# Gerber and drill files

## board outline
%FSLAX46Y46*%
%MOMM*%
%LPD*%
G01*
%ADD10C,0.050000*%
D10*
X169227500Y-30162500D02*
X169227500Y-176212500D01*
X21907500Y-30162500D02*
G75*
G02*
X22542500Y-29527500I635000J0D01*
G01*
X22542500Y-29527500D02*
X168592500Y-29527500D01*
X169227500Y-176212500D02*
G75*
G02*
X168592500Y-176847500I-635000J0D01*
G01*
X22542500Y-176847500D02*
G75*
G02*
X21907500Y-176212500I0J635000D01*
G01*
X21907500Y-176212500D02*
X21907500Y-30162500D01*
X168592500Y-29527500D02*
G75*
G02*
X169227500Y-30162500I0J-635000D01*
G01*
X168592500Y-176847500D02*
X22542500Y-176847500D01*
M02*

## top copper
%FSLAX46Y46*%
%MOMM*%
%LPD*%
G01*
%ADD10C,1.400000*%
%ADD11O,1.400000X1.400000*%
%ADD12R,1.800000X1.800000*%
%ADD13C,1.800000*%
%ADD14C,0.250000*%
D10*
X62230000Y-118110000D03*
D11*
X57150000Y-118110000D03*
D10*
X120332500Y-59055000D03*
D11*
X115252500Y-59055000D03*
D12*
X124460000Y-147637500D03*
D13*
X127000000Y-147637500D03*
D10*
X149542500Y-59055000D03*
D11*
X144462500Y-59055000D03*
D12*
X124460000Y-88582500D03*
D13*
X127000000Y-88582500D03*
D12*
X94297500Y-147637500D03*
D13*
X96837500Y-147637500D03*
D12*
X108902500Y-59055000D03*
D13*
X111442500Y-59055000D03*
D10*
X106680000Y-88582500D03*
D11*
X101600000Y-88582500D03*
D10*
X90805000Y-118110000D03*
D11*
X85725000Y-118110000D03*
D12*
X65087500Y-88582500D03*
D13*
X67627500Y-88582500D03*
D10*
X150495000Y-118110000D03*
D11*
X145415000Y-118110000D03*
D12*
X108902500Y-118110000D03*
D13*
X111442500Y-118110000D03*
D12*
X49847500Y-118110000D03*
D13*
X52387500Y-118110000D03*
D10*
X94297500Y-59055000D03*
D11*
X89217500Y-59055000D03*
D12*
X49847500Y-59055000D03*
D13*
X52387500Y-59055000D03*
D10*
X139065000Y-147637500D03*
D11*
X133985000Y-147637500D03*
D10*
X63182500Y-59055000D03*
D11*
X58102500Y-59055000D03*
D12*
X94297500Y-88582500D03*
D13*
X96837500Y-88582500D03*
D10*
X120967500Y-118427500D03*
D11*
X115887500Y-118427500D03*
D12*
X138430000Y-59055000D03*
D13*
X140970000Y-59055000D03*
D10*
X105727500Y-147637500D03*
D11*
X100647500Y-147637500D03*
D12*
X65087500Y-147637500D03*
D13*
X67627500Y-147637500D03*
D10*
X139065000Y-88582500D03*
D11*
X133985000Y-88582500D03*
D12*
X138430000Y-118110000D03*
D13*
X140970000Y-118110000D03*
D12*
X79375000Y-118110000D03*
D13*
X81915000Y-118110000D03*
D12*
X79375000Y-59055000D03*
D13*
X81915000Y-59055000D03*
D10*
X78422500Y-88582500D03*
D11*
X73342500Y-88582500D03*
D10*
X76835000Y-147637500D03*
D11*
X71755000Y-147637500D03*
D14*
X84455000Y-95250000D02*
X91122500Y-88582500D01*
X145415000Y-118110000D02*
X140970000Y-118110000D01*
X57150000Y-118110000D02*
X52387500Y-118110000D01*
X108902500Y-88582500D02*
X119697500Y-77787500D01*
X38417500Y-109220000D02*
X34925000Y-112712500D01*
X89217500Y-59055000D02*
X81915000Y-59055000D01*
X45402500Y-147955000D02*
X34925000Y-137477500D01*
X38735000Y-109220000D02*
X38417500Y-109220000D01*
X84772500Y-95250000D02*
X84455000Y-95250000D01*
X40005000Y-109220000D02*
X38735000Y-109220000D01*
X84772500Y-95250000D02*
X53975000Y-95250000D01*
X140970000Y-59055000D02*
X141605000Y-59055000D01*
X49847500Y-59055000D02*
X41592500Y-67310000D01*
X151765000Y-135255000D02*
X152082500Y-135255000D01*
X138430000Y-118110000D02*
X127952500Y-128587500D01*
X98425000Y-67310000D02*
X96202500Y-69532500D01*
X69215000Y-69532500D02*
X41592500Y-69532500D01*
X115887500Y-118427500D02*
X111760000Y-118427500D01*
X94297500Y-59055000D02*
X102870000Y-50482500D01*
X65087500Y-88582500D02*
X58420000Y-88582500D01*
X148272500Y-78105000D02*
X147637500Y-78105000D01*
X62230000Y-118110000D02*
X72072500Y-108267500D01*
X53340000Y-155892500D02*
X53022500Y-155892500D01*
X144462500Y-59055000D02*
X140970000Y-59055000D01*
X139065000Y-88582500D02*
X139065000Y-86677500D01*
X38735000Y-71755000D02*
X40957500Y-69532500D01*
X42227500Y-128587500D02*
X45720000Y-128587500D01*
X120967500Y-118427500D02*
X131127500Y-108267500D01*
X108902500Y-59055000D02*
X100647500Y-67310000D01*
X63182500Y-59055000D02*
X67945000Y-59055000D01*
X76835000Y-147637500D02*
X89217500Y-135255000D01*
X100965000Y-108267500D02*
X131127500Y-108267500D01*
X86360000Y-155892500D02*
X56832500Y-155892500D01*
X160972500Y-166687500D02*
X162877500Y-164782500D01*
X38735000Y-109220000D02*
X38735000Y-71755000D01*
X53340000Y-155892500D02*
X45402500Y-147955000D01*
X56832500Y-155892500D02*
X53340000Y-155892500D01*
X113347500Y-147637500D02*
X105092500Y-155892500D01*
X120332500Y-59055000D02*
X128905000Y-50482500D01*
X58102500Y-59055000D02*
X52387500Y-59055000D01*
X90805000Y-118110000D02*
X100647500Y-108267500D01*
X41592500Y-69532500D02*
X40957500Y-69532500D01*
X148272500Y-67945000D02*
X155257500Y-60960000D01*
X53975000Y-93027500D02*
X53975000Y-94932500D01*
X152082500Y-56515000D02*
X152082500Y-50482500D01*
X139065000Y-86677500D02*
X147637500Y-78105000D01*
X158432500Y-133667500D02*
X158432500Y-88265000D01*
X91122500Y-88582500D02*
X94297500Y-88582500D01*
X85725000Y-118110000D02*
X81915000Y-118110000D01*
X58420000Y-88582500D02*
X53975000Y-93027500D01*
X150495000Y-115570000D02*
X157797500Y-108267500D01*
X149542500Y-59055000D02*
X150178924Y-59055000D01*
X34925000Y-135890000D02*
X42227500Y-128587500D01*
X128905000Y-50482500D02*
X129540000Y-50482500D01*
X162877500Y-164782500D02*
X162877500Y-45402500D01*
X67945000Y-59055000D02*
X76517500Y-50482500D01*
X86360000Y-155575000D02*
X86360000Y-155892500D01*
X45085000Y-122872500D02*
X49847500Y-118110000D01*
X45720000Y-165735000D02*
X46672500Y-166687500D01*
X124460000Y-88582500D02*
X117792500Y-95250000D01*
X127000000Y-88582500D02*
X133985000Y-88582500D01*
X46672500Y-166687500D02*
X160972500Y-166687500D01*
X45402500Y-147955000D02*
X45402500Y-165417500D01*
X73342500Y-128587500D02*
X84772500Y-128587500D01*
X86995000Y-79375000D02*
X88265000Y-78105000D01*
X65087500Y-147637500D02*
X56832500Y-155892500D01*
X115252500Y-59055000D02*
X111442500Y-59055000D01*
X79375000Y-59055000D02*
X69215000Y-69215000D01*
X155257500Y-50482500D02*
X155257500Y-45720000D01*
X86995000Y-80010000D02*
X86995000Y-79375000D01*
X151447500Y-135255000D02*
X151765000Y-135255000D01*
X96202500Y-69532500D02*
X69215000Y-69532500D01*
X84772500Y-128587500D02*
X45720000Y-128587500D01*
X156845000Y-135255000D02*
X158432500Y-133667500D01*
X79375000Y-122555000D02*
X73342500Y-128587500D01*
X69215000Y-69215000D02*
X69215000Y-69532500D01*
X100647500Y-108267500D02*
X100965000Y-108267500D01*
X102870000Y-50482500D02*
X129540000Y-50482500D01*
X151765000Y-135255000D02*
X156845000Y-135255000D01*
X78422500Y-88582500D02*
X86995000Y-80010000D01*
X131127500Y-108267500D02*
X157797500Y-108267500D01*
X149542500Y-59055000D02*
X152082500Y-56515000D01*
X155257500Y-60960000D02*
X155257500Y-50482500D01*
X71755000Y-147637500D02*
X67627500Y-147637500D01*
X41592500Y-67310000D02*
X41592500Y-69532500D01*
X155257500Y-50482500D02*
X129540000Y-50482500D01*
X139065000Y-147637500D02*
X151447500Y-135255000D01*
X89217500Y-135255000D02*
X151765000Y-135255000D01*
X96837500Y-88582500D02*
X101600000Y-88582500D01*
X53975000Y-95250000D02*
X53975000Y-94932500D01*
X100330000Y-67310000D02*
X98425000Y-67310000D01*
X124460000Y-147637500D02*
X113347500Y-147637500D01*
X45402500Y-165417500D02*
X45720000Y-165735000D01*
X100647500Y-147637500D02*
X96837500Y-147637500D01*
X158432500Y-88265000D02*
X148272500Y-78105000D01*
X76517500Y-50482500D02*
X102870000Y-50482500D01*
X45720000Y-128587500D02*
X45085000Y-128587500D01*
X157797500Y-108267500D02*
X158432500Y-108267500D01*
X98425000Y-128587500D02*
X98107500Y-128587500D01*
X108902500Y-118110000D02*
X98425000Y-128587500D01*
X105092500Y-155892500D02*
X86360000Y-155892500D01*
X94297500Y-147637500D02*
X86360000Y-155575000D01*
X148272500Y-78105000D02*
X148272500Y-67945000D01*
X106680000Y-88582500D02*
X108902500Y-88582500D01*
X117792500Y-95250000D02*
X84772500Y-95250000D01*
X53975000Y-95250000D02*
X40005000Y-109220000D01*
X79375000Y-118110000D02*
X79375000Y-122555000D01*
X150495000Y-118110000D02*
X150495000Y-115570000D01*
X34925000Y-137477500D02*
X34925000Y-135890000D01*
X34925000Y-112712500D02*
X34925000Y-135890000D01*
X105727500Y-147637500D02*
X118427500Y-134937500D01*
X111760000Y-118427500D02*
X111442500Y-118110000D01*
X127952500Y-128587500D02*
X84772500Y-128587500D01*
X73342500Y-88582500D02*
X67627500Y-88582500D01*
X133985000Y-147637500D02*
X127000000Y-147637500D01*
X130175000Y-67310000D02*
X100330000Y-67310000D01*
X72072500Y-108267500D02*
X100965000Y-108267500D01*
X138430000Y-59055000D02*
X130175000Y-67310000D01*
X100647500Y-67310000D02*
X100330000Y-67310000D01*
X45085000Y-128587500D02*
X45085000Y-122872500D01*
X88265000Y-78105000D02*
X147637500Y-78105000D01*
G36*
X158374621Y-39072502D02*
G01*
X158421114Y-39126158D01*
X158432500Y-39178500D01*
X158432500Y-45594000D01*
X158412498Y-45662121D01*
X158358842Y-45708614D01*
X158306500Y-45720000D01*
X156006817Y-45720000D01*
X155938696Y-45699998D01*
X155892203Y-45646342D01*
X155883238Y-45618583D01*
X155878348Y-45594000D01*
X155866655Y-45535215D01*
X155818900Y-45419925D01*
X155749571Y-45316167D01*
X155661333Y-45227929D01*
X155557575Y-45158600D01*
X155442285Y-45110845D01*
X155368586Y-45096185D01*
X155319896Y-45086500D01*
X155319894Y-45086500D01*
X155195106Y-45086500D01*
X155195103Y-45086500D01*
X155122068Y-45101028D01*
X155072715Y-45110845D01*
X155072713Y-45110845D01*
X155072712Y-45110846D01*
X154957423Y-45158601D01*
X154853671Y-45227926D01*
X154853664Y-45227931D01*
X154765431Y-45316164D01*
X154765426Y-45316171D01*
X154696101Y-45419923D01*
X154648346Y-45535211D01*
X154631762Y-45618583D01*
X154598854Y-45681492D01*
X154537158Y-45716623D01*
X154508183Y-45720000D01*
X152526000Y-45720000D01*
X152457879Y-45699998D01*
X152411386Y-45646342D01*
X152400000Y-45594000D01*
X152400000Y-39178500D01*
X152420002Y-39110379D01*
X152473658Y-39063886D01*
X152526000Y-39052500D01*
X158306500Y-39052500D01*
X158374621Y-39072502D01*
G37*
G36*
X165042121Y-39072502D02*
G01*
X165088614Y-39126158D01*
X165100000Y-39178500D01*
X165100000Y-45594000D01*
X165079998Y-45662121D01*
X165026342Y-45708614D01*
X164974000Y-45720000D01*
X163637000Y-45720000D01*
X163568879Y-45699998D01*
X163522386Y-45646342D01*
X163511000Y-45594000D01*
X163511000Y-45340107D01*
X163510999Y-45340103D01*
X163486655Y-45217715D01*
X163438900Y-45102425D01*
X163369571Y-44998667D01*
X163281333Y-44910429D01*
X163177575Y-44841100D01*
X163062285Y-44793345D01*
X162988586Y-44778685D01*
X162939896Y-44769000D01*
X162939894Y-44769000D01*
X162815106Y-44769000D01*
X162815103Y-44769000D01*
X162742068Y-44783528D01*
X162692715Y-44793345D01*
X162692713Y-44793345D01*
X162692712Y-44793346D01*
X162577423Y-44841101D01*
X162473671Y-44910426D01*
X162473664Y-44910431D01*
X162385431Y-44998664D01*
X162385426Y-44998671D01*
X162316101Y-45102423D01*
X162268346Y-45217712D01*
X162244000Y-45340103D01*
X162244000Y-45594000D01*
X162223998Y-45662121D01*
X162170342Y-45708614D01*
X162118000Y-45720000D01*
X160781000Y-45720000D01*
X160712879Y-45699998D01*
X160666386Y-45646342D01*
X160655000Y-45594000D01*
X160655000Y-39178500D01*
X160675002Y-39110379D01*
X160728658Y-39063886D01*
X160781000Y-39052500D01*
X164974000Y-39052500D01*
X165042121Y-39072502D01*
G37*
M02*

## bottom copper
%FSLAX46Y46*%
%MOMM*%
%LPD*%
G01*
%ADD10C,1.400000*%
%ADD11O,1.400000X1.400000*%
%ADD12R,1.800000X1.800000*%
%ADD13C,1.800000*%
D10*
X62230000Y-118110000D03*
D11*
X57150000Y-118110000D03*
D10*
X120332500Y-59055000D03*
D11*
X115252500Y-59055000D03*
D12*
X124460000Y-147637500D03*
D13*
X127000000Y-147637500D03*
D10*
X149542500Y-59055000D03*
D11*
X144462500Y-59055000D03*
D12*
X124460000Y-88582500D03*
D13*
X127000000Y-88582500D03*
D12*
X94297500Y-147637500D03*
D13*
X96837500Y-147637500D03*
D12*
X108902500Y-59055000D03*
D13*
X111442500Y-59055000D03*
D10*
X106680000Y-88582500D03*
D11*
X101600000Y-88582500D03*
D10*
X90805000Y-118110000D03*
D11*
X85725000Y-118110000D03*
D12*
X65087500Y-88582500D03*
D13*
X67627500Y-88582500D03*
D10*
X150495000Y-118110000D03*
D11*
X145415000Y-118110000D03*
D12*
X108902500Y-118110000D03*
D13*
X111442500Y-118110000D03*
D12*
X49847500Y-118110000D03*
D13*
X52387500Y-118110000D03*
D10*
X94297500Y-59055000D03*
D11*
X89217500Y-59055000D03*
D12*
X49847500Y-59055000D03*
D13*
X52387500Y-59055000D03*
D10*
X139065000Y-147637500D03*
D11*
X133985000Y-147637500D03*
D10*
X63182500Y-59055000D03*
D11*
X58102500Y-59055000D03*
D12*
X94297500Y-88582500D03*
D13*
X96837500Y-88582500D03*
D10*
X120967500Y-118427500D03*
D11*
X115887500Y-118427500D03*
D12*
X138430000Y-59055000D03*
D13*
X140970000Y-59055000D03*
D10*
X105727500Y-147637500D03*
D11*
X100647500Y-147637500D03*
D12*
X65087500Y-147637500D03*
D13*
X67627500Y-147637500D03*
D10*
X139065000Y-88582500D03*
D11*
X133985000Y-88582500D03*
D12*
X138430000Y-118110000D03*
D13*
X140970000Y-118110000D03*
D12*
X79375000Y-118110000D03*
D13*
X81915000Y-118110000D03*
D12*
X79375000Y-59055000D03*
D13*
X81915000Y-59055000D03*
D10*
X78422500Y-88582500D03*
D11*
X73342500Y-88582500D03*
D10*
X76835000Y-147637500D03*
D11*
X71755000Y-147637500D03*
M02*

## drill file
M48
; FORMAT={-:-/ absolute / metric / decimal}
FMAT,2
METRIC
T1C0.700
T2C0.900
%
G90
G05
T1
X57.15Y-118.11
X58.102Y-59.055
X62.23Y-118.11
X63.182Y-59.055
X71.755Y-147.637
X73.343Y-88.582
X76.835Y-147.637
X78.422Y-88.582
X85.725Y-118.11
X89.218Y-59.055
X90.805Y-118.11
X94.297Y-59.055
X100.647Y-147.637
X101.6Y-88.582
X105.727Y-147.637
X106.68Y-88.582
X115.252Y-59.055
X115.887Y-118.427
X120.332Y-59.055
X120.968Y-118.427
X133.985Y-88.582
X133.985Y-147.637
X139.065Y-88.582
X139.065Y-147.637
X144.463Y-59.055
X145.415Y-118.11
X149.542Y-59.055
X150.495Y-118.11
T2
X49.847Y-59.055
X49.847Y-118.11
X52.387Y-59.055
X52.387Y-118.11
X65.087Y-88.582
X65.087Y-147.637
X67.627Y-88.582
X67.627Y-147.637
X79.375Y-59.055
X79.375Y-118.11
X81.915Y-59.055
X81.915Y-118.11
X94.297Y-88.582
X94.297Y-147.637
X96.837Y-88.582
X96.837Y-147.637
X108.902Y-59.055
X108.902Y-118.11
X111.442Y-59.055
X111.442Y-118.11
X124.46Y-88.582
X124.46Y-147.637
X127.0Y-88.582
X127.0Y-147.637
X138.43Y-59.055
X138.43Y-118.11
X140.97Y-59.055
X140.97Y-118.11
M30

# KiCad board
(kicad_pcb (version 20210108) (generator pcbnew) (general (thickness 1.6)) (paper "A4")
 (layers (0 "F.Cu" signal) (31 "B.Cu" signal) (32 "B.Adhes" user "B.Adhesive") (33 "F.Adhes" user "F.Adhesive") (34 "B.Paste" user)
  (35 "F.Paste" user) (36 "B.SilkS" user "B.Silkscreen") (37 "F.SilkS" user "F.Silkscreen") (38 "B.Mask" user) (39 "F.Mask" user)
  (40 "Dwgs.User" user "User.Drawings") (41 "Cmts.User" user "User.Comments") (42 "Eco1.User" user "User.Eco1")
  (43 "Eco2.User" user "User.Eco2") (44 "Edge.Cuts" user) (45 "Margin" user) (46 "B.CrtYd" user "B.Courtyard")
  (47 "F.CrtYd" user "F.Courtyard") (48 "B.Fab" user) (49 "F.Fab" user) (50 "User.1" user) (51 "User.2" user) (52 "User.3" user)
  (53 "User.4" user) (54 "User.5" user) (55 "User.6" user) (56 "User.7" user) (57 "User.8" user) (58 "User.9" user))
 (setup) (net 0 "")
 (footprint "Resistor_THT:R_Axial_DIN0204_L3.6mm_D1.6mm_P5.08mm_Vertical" (layer "F.Cu") (at 62.23 118.11 180)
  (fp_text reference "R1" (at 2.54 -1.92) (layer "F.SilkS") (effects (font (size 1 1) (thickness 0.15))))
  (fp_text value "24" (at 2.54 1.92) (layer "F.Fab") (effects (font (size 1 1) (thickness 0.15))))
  (pad "1" thru_hole circle (at 0 0 180) (locked) (size 1.4 1.4) (drill 0.7) (layers *.Cu *.Mask))
  (pad "2" thru_hole oval (at 5.08 0 180) (locked) (size 1.4 1.4) (drill 0.7) (layers *.Cu *.Mask)))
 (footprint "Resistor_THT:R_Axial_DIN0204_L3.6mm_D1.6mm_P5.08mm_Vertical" (layer "F.Cu") (at 120.3325 59.055 180)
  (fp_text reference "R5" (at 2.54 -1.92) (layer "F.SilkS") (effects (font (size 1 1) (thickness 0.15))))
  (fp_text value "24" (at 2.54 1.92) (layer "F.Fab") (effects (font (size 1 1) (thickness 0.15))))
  (pad "1" thru_hole circle (at 0 0 180) (locked) (size 1.4 1.4) (drill 0.7) (layers *.Cu *.Mask))
  (pad "2" thru_hole oval (at 5.08 0 180) (locked) (size 1.4 1.4) (drill 0.7) (layers *.Cu *.Mask)))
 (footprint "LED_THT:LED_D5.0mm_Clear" (layer "F.Cu") (at 124.46 147.6375)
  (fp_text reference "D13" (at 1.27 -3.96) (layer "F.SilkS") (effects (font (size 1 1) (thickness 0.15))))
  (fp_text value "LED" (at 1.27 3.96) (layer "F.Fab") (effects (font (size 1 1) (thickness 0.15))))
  (pad "1" thru_hole rect (at 0 0) (locked) (size 1.8 1.8) (drill 0.9) (layers *.Cu *.Mask))
  (pad "2" thru_hole circle (at 2.54 0) (locked) (size 1.8 1.8) (drill 0.9) (layers *.Cu *.Mask)))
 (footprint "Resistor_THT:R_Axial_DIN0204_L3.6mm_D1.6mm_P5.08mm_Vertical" (layer "F.Cu") (at 149.5425 59.055 180)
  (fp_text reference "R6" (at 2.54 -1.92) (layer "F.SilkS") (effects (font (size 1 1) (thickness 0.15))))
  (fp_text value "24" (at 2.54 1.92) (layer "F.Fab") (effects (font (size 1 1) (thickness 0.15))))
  (pad "1" thru_hole circle (at 0 0 180) (locked) (size 1.4 1.4) (drill 0.7) (layers *.Cu *.Mask))
  (pad "2" thru_hole oval (at 5.08 0 180) (locked) (size 1.4 1.4) (drill 0.7) (layers *.Cu *.Mask)))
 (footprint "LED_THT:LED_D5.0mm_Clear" (layer "F.Cu") (at 124.46 88.5825)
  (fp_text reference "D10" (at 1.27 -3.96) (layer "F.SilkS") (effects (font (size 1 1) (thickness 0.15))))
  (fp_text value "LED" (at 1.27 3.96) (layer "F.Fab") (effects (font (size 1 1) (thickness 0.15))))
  (pad "1" thru_hole rect (at 0 0) (locked) (size 1.8 1.8) (drill 0.9) (layers *.Cu *.Mask))
  (pad "2" thru_hole circle (at 2.54 0) (locked) (size 1.8 1.8) (drill 0.9) (layers *.Cu *.Mask)))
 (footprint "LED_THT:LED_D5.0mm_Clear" (layer "F.Cu") (at 94.2975 147.6375)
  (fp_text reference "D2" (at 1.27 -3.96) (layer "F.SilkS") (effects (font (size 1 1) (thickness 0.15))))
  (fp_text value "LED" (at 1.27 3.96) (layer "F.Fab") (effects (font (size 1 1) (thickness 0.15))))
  (pad "1" thru_hole rect (at 0 0) (locked) (size 1.8 1.8) (drill 0.9) (layers *.Cu *.Mask))
  (pad "2" thru_hole circle (at 2.54 0) (locked) (size 1.8 1.8) (drill 0.9) (layers *.Cu *.Mask)))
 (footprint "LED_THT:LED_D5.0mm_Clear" (layer "F.Cu") (at 108.9025 59.055)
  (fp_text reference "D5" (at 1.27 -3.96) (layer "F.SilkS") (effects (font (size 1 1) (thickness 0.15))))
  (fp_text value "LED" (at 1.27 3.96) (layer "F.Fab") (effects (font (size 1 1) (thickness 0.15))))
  (pad "1" thru_hole rect (at 0 0) (locked) (size 1.8 1.8) (drill 0.9) (layers *.Cu *.Mask))
  (pad "2" thru_hole circle (at 2.54 0) (locked) (size 1.8 1.8) (drill 0.9) (layers *.Cu *.Mask)))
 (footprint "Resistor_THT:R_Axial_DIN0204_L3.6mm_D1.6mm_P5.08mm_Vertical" (layer "F.Cu") (at 106.68 88.5825 180)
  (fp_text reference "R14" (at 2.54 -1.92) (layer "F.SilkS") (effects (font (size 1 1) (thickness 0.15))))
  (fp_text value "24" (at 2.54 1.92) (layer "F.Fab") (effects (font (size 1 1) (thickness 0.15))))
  (pad "1" thru_hole circle (at 0 0 180) (locked) (size 1.4 1.4) (drill 0.7) (layers *.Cu *.Mask))
  (pad "2" thru_hole oval (at 5.08 0 180) (locked) (size 1.4 1.4) (drill 0.7) (layers *.Cu *.Mask)))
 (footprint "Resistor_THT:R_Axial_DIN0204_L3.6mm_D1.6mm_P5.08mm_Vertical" (layer "F.Cu") (at 90.805 118.11 180)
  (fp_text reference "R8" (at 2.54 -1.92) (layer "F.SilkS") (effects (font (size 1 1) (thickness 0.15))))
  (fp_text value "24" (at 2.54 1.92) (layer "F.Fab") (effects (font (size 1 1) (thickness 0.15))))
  (pad "1" thru_hole circle (at 0 0 180) (locked) (size 1.4 1.4) (drill 0.7) (layers *.Cu *.Mask))
  (pad "2" thru_hole oval (at 5.08 0 180) (locked) (size 1.4 1.4) (drill 0.7) (layers *.Cu *.Mask)))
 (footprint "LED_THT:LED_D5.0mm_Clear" (layer "F.Cu") (at 65.0875 88.5825)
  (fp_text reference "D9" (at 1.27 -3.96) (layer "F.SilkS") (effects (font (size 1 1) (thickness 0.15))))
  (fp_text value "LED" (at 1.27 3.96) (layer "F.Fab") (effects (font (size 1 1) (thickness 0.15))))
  (pad "1" thru_hole rect (at 0 0) (locked) (size 1.8 1.8) (drill 0.9) (layers *.Cu *.Mask))
  (pad "2" thru_hole circle (at 2.54 0) (locked) (size 1.8 1.8) (drill 0.9) (layers *.Cu *.Mask)))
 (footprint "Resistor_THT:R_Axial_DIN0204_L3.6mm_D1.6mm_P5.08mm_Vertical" (layer "F.Cu") (at 150.495 118.11 180)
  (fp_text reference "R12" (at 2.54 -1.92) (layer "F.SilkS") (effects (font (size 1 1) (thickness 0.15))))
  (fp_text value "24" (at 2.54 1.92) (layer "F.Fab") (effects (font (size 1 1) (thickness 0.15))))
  (pad "1" thru_hole circle (at 0 0 180) (locked) (size 1.4 1.4) (drill 0.7) (layers *.Cu *.Mask))
  (pad "2" thru_hole oval (at 5.08 0 180) (locked) (size 1.4 1.4) (drill 0.7) (layers *.Cu *.Mask)))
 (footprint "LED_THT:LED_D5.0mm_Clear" (layer "F.Cu") (at 108.9025 118.11)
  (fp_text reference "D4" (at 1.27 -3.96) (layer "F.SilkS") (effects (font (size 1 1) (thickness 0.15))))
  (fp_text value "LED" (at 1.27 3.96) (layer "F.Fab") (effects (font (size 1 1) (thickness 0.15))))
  (pad "1" thru_hole rect (at 0 0) (locked) (size 1.8 1.8) (drill 0.9) (layers *.Cu *.Mask))
  (pad "2" thru_hole circle (at 2.54 0) (locked) (size 1.8 1.8) (drill 0.9) (layers *.Cu *.Mask)))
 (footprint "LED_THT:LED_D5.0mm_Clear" (layer "F.Cu") (at 49.8475 118.11)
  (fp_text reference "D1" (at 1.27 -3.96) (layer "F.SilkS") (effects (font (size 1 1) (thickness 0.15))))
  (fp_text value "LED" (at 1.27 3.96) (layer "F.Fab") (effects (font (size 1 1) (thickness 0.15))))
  (pad "1" thru_hole rect (at 0 0) (locked) (size 1.8 1.8) (drill 0.9) (layers *.Cu *.Mask))
  (pad "2" thru_hole circle (at 2.54 0) (locked) (size 1.8 1.8) (drill 0.9) (layers *.Cu *.Mask)))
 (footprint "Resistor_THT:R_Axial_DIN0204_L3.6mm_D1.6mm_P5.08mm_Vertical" (layer "F.Cu") (at 94.2975 59.055 180)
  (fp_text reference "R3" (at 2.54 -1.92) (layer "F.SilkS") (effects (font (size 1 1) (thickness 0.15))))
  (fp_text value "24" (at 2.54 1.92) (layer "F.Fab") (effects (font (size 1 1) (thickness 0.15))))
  (pad "1" thru_hole circle (at 0 0 180) (locked) (size 1.4 1.4) (drill 0.7) (layers *.Cu *.Mask))
  (pad "2" thru_hole oval (at 5.08 0 180) (locked) (size 1.4 1.4) (drill 0.7) (layers *.Cu *.Mask)))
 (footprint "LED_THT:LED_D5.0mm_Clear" (layer "F.Cu") (at 49.8475 59.055)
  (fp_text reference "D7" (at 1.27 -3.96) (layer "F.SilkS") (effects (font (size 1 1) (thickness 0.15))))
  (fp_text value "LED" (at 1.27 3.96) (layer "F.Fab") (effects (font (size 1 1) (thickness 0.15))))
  (pad "1" thru_hole rect (at 0 0) (locked) (size 1.8 1.8) (drill 0.9) (layers *.Cu *.Mask))
  (pad "2" thru_hole circle (at 2.54 0) (locked) (size 1.8 1.8) (drill 0.9) (layers *.Cu *.Mask)))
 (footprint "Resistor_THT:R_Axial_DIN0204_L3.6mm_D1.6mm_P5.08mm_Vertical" (layer "F.Cu") (at 139.065 147.6375 180)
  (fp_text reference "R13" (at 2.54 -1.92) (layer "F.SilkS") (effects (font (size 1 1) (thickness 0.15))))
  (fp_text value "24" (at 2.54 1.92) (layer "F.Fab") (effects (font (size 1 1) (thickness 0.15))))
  (pad "1" thru_hole circle (at 0 0 180) (locked) (size 1.4 1.4) (drill 0.7) (layers *.Cu *.Mask))
  (pad "2" thru_hole oval (at 5.08 0 180) (locked) (size 1.4 1.4) (drill 0.7) (layers *.Cu *.Mask)))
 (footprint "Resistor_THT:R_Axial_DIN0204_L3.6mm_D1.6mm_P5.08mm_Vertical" (layer "F.Cu") (at 63.1825 59.055 180)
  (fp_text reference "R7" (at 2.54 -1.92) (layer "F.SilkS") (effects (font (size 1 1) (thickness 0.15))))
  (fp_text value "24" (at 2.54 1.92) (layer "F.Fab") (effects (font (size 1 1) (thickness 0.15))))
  (pad "1" thru_hole circle (at 0 0 180) (locked) (size 1.4 1.4) (drill 0.7) (layers *.Cu *.Mask))
  (pad "2" thru_hole oval (at 5.08 0 180) (locked) (size 1.4 1.4) (drill 0.7) (layers *.Cu *.Mask)))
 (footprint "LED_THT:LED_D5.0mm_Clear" (layer "F.Cu") (at 94.2975 88.5825)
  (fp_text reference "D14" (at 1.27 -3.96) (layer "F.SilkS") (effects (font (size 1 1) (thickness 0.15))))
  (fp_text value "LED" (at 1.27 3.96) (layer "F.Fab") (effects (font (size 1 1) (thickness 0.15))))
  (pad "1" thru_hole rect (at 0 0) (locked) (size 1.8 1.8) (drill 0.9) (layers *.Cu *.Mask))
  (pad "2" thru_hole circle (at 2.54 0) (locked) (size 1.8 1.8) (drill 0.9) (layers *.Cu *.Mask)))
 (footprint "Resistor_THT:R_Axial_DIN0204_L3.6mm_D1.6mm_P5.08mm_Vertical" (layer "F.Cu") (at 120.9675 118.4275 180)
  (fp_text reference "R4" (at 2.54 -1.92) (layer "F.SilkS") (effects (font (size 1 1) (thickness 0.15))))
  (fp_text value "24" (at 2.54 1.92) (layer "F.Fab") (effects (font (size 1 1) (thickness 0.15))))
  (pad "1" thru_hole circle (at 0 0 180) (locked) (size 1.4 1.4) (drill 0.7) (layers *.Cu *.Mask))
  (pad "2" thru_hole oval (at 5.08 0 180) (locked) (size 1.4 1.4) (drill 0.7) (layers *.Cu *.Mask)))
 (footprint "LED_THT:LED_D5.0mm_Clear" (layer "F.Cu") (at 138.43 59.055)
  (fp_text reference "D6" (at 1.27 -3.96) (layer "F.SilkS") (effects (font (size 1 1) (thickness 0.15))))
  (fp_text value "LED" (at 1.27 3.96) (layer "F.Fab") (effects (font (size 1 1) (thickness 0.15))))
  (pad "1" thru_hole rect (at 0 0) (locked) (size 1.8 1.8) (drill 0.9) (layers *.Cu *.Mask))
  (pad "2" thru_hole circle (at 2.54 0) (locked) (size 1.8 1.8) (drill 0.9) (layers *.Cu *.Mask)))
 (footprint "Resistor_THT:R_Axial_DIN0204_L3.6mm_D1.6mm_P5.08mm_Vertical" (layer "F.Cu") (at 105.7275 147.6375 180)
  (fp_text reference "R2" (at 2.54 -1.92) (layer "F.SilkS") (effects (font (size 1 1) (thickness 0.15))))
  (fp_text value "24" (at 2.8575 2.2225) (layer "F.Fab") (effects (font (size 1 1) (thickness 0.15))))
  (pad "1" thru_hole circle (at 0 0 180) (locked) (size 1.4 1.4) (drill 0.7) (layers *.Cu *.Mask))
  (pad "2" thru_hole oval (at 5.08 0 180) (locked) (size 1.4 1.4) (drill 0.7) (layers *.Cu *.Mask)))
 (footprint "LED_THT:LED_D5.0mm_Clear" (layer "F.Cu") (at 65.0875 147.6375)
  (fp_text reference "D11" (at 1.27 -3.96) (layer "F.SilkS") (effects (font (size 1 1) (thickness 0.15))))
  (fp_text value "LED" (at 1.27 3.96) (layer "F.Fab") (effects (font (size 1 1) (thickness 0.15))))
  (pad "1" thru_hole rect (at 0 0) (locked) (size 1.8 1.8) (drill 0.9) (layers *.Cu *.Mask))
  (pad "2" thru_hole circle (at 2.54 0) (locked) (size 1.8 1.8) (drill 0.9) (layers *.Cu *.Mask)))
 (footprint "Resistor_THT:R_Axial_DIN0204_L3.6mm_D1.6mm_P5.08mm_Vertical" (layer "F.Cu") (at 139.065 88.5825 180)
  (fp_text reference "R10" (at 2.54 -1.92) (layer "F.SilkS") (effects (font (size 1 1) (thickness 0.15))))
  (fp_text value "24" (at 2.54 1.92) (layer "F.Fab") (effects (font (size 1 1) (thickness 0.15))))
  (pad "1" thru_hole circle (at 0 0 180) (locked) (size 1.4 1.4) (drill 0.7) (layers *.Cu *.Mask))
  (pad "2" thru_hole oval (at 5.08 0 180) (locked) (size 1.4 1.4) (drill 0.7) (layers *.Cu *.Mask)))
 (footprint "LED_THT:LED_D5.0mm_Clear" (layer "F.Cu") (at 138.43 118.11)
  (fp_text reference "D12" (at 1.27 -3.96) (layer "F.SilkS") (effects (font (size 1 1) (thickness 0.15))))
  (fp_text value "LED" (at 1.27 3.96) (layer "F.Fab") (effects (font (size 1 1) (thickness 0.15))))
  (pad "1" thru_hole rect (at 0 0) (locked) (size 1.8 1.8) (drill 0.9) (layers *.Cu *.Mask))
  (pad "2" thru_hole circle (at 2.54 0) (locked) (size 1.8 1.8) (drill 0.9) (layers *.Cu *.Mask)))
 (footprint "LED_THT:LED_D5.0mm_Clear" (layer "F.Cu") (at 79.375 118.11)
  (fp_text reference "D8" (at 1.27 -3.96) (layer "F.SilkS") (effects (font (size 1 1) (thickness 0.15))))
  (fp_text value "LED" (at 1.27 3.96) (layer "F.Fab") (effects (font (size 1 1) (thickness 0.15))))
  (pad "1" thru_hole rect (at 0 0) (locked) (size 1.8 1.8) (drill 0.9) (layers *.Cu *.Mask))
  (pad "2" thru_hole circle (at 2.54 0) (locked) (size 1.8 1.8) (drill 0.9) (layers *.Cu *.Mask)))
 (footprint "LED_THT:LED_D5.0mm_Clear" (layer "F.Cu") (at 79.375 59.055)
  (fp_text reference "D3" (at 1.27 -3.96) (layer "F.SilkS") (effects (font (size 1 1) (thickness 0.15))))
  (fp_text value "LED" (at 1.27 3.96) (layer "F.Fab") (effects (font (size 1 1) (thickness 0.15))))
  (pad "1" thru_hole rect (at 0 0) (locked) (size 1.8 1.8) (drill 0.9) (layers *.Cu *.Mask))
  (pad "2" thru_hole circle (at 2.54 0) (locked) (size 1.8 1.8) (drill 0.9) (layers *.Cu *.Mask)))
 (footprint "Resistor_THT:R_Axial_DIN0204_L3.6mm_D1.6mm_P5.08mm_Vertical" (layer "F.Cu") (at 78.4225 88.5825 180)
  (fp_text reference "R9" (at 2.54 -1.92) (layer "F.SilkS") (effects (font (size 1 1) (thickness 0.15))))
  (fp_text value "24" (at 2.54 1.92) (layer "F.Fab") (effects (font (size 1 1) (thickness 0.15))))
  (pad "1" thru_hole circle (at 0 0 180) (locked) (size 1.4 1.4) (drill 0.7) (layers *.Cu *.Mask))
  (pad "2" thru_hole oval (at 5.08 0 180) (locked) (size 1.4 1.4) (drill 0.7) (layers *.Cu *.Mask)))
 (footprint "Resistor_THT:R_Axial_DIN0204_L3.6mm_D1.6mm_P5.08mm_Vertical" (layer "F.Cu") (at 76.835 147.6375 180)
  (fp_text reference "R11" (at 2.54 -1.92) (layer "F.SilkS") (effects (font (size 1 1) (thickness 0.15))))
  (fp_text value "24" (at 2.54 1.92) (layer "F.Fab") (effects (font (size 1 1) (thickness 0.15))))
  (pad "1" thru_hole circle (at 0 0 180) (locked) (size 1.4 1.4) (drill 0.7) (layers *.Cu *.Mask))
  (pad "2" thru_hole oval (at 5.08 0 180) (locked) (size 1.4 1.4) (drill 0.7) (layers *.Cu *.Mask)))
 (gr_line (start 169.2275 30.1625) (end 169.2275 176.2125) (layer "Edge.Cuts") (width 0.05))
 (gr_arc (start 22.5425 30.1625) (end 22.5425 29.5275) (angle -90) (layer "Edge.Cuts") (width 0.05))
 (gr_line (start 22.5425 29.5275) (end 168.5925 29.5275) (layer "Edge.Cuts") (width 0.05))
 (gr_arc (start 168.5925 176.2125) (end 168.5925 176.8475) (angle -90) (layer "Edge.Cuts") (width 0.05))
 (gr_arc (start 22.5425 176.2125) (end 22.5425 176.8475) (angle 90) (layer "Edge.Cuts") (width 0.05))
 (gr_line (start 21.9075 176.2125) (end 21.9075 30.1625) (layer "Edge.Cuts") (width 0.05))
 (gr_arc (start 168.5925 30.1625) (end 169.2275 30.1625) (angle -90) (layer "Edge.Cuts") (width 0.05))
 (gr_line (start 168.5925 176.8475) (end 22.5425 176.8475) (layer "Edge.Cuts") (width 0.05))
 (segment (start 84.455 95.25) (end 91.1225 88.5825) (width 0.25) (layer "F.Cu") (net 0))
 (segment (start 145.415 118.11) (end 140.97 118.11) (width 0.25) (layer "F.Cu") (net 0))
 (segment (start 57.15 118.11) (end 52.3875 118.11) (width 0.25) (layer "F.Cu") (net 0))
 (segment (start 108.9025 88.5825) (end 119.6975 77.7875) (width 0.25) (layer "F.Cu") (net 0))
 (segment (start 38.4175 109.22) (end 34.925 112.7125) (width 0.25) (layer "F.Cu") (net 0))
 (segment (start 89.2175 59.055) (end 81.915 59.055) (width 0.25) (layer "F.Cu") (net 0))
 (segment (start 45.4025 147.955) (end 34.925 137.4775) (width 0.25) (layer "F.Cu") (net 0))
 (segment (start 38.735 109.22) (end 38.4175 109.22) (width 0.25) (layer "F.Cu") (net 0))
 (segment (start 84.7725 95.25) (end 84.455 95.25) (width 0.25) (layer "F.Cu") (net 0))
 (segment (start 40.005 109.22) (end 38.735 109.22) (width 0.25) (layer "F.Cu") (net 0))
 (segment (start 84.7725 95.25) (end 53.975 95.25) (width 0.25) (layer "F.Cu") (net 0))
 (segment (start 140.97 59.055) (end 141.605 59.055) (width 0.25) (layer "F.Cu") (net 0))
 (segment (start 49.8475 59.055) (end 41.5925 67.31) (width 0.25) (layer "F.Cu") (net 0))
 (segment (start 151.765 135.255) (end 152.0825 135.255) (width 0.25) (layer "F.Cu") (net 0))
 (segment (start 138.43 118.11) (end 127.9525 128.5875) (width 0.25) (layer "F.Cu") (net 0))
 (segment (start 98.425 67.31) (end 96.2025 69.5325) (width 0.25) (layer "F.Cu") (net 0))
 (segment (start 69.215 69.5325) (end 41.5925 69.5325) (width 0.25) (layer "F.Cu") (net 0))
 (segment (start 115.8875 118.4275) (end 111.76 118.4275) (width 0.25) (layer "F.Cu") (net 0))
 (segment (start 94.2975 59.055) (end 102.87 50.4825) (width 0.25) (layer "F.Cu") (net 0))
 (segment (start 65.0875 88.5825) (end 58.42 88.5825) (width 0.25) (layer "F.Cu") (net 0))
 (segment (start 148.2725 78.105) (end 147.6375 78.105) (width 0.25) (layer "F.Cu") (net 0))
 (segment (start 62.23 118.11) (end 72.0725 108.2675) (width 0.25) (layer "F.Cu") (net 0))
 (segment (start 53.34 155.8925) (end 53.0225 155.8925) (width 0.25) (layer "F.Cu") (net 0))
 (segment (start 144.4625 59.055) (end 140.97 59.055) (width 0.25) (layer "F.Cu") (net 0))
 (segment (start 139.065 88.5825) (end 139.065 86.6775) (width 0.25) (layer "F.Cu") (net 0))
 (segment (start 38.735 71.755) (end 40.9575 69.5325) (width 0.25) (layer "F.Cu") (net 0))
 (segment (start 42.2275 128.5875) (end 45.72 128.5875) (width 0.25) (layer "F.Cu") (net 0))
 (segment (start 120.9675 118.4275) (end 131.1275 108.2675) (width 0.25) (layer "F.Cu") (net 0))
 (segment (start 108.9025 59.055) (end 100.6475 67.31) (width 0.25) (layer "F.Cu") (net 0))
 (segment (start 63.1825 59.055) (end 67.945 59.055) (width 0.25) (layer "F.Cu") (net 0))
 (segment (start 76.835 147.6375) (end 89.2175 135.255) (width 0.25) (layer "F.Cu") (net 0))
 (segment (start 100.965 108.2675) (end 131.1275 108.2675) (width 0.25) (layer "F.Cu") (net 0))
 (segment (start 86.36 155.8925) (end 56.8325 155.8925) (width 0.25) (layer "F.Cu") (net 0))
 (segment (start 160.9725 166.6875) (end 162.8775 164.7825) (width 0.25) (layer "F.Cu") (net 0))
 (segment (start 38.735 109.22) (end 38.735 71.755) (width 0.25) (layer "F.Cu") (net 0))
 (segment (start 53.34 155.8925) (end 45.4025 147.955) (width 0.25) (layer "F.Cu") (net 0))
 (segment (start 56.8325 155.8925) (end 53.34 155.8925) (width 0.25) (layer "F.Cu") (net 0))
 (segment (start 113.3475 147.6375) (end 105.0925 155.8925) (width 0.25) (layer "F.Cu") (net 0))
 (segment (start 120.3325 59.055) (end 128.905 50.4825) (width 0.25) (layer "F.Cu") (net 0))
 (segment (start 58.1025 59.055) (end 52.3875 59.055) (width 0.25) (layer "F.Cu") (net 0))
 (segment (start 90.805 118.11) (end 100.6475 108.2675) (width 0.25) (layer "F.Cu") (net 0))
 (segment (start 41.5925 69.5325) (end 40.9575 69.5325) (width 0.25) (layer "F.Cu") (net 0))
 (segment (start 148.2725 67.945) (end 155.2575 60.96) (width 0.25) (layer "F.Cu") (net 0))
 (segment (start 53.975 93.0275) (end 53.975 94.9325) (width 0.25) (layer "F.Cu") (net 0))
 (segment (start 152.0825 56.515) (end 152.0825 50.4825) (width 0.25) (layer "F.Cu") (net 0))
 (segment (start 139.065 86.6775) (end 147.6375 78.105) (width 0.25) (layer "F.Cu") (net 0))
 (segment (start 158.4325 133.6675) (end 158.4325 88.265) (width 0.25) (layer "F.Cu") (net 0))
 (segment (start 91.1225 88.5825) (end 94.2975 88.5825) (width 0.25) (layer "F.Cu") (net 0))
 (segment (start 85.725 118.11) (end 81.915 118.11) (width 0.25) (layer "F.Cu") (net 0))
 (segment (start 58.42 88.5825) (end 53.975 93.0275) (width 0.25) (layer "F.Cu") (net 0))
 (segment (start 150.495 115.57) (end 157.7975 108.2675) (width 0.25) (layer "F.Cu") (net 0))
 (segment (start 149.5425 59.055) (end 150.178924 59.055) (width 0.25) (layer "F.Cu") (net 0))
 (segment (start 34.925 135.89) (end 42.2275 128.5875) (width 0.25) (layer "F.Cu") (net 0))
 (segment (start 128.905 50.4825) (end 129.54 50.4825) (width 0.25) (layer "F.Cu") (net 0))
 (segment (start 162.8775 164.7825) (end 162.8775 45.4025) (width 0.25) (layer "F.Cu") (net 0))
 (segment (start 67.945 59.055) (end 76.5175 50.4825) (width 0.25) (layer "F.Cu") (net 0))
 (segment (start 86.36 155.575) (end 86.36 155.8925) (width 0.25) (layer "F.Cu") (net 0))
 (segment (start 45.085 122.8725) (end 49.8475 118.11) (width 0.25) (layer "F.Cu") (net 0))
 (segment (start 45.72 165.735) (end 46.6725 166.6875) (width 0.25) (layer "F.Cu") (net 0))
 (segment (start 124.46 88.5825) (end 117.7925 95.25) (width 0.25) (layer "F.Cu") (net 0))
 (segment (start 127 88.5825) (end 133.985 88.5825) (width 0.25) (layer "F.Cu") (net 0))
 (segment (start 46.6725 166.6875) (end 160.9725 166.6875) (width 0.25) (layer "F.Cu") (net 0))
 (segment (start 45.4025 147.955) (end 45.4025 165.4175) (width 0.25) (layer "F.Cu") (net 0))
 (segment (start 73.3425 128.5875) (end 84.7725 128.5875) (width 0.25) (layer "F.Cu") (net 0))
 (segment (start 86.995 79.375) (end 88.265 78.105) (width 0.25) (layer "F.Cu") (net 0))
 (segment (start 65.0875 147.6375) (end 56.8325 155.8925) (width 0.25) (layer "F.Cu") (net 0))
 (segment (start 115.2525 59.055) (end 111.4425 59.055) (width 0.25) (layer "F.Cu") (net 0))
 (segment (start 79.375 59.055) (end 69.215 69.215) (width 0.25) (layer "F.Cu") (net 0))
 (segment (start 155.2575 50.4825) (end 155.2575 45.72) (width 0.25) (layer "F.Cu") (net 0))
 (segment (start 86.995 80.01) (end 86.995 79.375) (width 0.25) (layer "F.Cu") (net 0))
 (segment (start 151.4475 135.255) (end 151.765 135.255) (width 0.25) (layer "F.Cu") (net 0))
 (segment (start 96.2025 69.5325) (end 69.215 69.5325) (width 0.25) (layer "F.Cu") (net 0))
 (segment (start 84.7725 128.5875) (end 45.72 128.5875) (width 0.25) (layer "F.Cu") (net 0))
 (segment (start 156.845 135.255) (end 158.4325 133.6675) (width 0.25) (layer "F.Cu") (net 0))
 (segment (start 79.375 122.555) (end 73.3425 128.5875) (width 0.25) (layer "F.Cu") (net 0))
 (segment (start 69.215 69.215) (end 69.215 69.5325) (width 0.25) (layer "F.Cu") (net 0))
 (segment (start 100.6475 108.2675) (end 100.965 108.2675) (width 0.25) (layer "F.Cu") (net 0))
 (segment (start 102.87 50.4825) (end 129.54 50.4825) (width 0.25) (layer "F.Cu") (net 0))
 (segment (start 151.765 135.255) (end 156.845 135.255) (width 0.25) (layer "F.Cu") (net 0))
 (segment (start 78.4225 88.5825) (end 86.995 80.01) (width 0.25) (layer "F.Cu") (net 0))
 (segment (start 131.1275 108.2675) (end 157.7975 108.2675) (width 0.25) (layer "F.Cu") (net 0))
 (segment (start 149.5425 59.055) (end 152.0825 56.515) (width 0.25) (layer "F.Cu") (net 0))
 (segment (start 155.2575 60.96) (end 155.2575 50.4825) (width 0.25) (layer "F.Cu") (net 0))
 (segment (start 71.755 147.6375) (end 67.6275 147.6375) (width 0.25) (layer "F.Cu") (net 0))
 (segment (start 41.5925 67.31) (end 41.5925 69.5325) (width 0.25) (layer "F.Cu") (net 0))
 (segment (start 155.2575 50.4825) (end 129.54 50.4825) (width 0.25) (layer "F.Cu") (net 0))
 (segment (start 139.065 147.6375) (end 151.4475 135.255) (width 0.25) (layer "F.Cu") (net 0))
 (segment (start 89.2175 135.255) (end 151.765 135.255) (width 0.25) (layer "F.Cu") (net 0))
 (segment (start 96.8375 88.5825) (end 101.6 88.5825) (width 0.25) (layer "F.Cu") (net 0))
 (segment (start 53.975 95.25) (end 53.975 94.9325) (width 0.25) (layer "F.Cu") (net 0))
 (segment (start 100.33 67.31) (end 98.425 67.31) (width 0.25) (layer "F.Cu") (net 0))
 (segment (start 124.46 147.6375) (end 113.3475 147.6375) (width 0.25) (layer "F.Cu") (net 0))
 (segment (start 45.4025 165.4175) (end 45.72 165.735) (width 0.25) (layer "F.Cu") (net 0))
 (segment (start 100.6475 147.6375) (end 96.8375 147.6375) (width 0.25) (layer "F.Cu") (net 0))
 (segment (start 158.4325 88.265) (end 148.2725 78.105) (width 0.25) (layer "F.Cu") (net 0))
 (segment (start 76.5175 50.4825) (end 102.87 50.4825) (width 0.25) (layer "F.Cu") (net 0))
 (segment (start 45.72 128.5875) (end 45.085 128.5875) (width 0.25) (layer "F.Cu") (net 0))
 (segment (start 157.7975 108.2675) (end 158.4325 108.2675) (width 0.25) (layer "F.Cu") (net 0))
 (segment (start 98.425 128.5875) (end 98.1075 128.5875) (width 0.25) (layer "F.Cu") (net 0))
 (segment (start 108.9025 118.11) (end 98.425 128.5875) (width 0.25) (layer "F.Cu") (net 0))
 (segment (start 105.0925 155.8925) (end 86.36 155.8925) (width 0.25) (layer "F.Cu") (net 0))
 (segment (start 94.2975 147.6375) (end 86.36 155.575) (width 0.25) (layer "F.Cu") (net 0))
 (segment (start 148.2725 78.105) (end 148.2725 67.945) (width 0.25) (layer "F.Cu") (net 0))
 (segment (start 106.68 88.5825) (end 108.9025 88.5825) (width 0.25) (layer "F.Cu") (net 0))
 (segment (start 117.7925 95.25) (end 84.7725 95.25) (width 0.25) (layer "F.Cu") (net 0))
 (segment (start 53.975 95.25) (end 40.005 109.22) (width 0.25) (layer "F.Cu") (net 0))
 (segment (start 79.375 118.11) (end 79.375 122.555) (width 0.25) (layer "F.Cu") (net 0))
 (segment (start 150.495 118.11) (end 150.495 115.57) (width 0.25) (layer "F.Cu") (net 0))
 (segment (start 34.925 137.4775) (end 34.925 135.89) (width 0.25) (layer "F.Cu") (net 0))
 (segment (start 34.925 112.7125) (end 34.925 135.89) (width 0.25) (layer "F.Cu") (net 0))
 (segment (start 105.7275 147.6375) (end 118.4275 134.9375) (width 0.25) (layer "F.Cu") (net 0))
 (segment (start 111.76 118.4275) (end 111.4425 118.11) (width 0.25) (layer "F.Cu") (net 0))
 (segment (start 127.9525 128.5875) (end 84.7725 128.5875) (width 0.25) (layer "F.Cu") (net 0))
 (segment (start 73.3425 88.5825) (end 67.6275 88.5825) (width 0.25) (layer "F.Cu") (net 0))
 (segment (start 133.985 147.6375) (end 127 147.6375) (width 0.25) (layer "F.Cu") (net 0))
 (segment (start 130.175 67.31) (end 100.33 67.31) (width 0.25) (layer "F.Cu") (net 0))
 (segment (start 72.0725 108.2675) (end 100.965 108.2675) (width 0.25) (layer "F.Cu") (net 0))
 (segment (start 138.43 59.055) (end 130.175 67.31) (width 0.25) (layer "F.Cu") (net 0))
 (segment (start 100.6475 67.31) (end 100.33 67.31) (width 0.25) (layer "F.Cu") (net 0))
 (segment (start 45.085 128.5875) (end 45.085 122.8725) (width 0.25) (layer "F.Cu") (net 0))
 (segment (start 88.265 78.105) (end 147.6375 78.105) (width 0.25) (layer "F.Cu") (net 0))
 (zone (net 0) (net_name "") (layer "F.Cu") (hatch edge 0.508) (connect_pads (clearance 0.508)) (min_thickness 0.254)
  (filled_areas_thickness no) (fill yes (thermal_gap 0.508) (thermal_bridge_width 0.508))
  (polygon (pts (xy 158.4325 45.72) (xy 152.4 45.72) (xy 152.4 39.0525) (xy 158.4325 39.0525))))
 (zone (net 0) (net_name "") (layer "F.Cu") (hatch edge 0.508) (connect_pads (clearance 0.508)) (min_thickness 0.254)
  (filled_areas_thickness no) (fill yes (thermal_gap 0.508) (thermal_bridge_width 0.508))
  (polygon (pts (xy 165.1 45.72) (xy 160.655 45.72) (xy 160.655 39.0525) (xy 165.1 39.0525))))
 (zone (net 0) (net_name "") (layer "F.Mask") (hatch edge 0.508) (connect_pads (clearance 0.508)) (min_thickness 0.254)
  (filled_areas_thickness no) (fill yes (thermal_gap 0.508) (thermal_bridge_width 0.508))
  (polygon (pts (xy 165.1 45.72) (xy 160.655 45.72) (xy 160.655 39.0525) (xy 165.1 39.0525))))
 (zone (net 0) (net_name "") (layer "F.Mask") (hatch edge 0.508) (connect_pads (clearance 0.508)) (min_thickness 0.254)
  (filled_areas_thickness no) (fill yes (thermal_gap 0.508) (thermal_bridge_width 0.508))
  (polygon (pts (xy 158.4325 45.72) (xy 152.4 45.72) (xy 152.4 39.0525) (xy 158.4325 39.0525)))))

